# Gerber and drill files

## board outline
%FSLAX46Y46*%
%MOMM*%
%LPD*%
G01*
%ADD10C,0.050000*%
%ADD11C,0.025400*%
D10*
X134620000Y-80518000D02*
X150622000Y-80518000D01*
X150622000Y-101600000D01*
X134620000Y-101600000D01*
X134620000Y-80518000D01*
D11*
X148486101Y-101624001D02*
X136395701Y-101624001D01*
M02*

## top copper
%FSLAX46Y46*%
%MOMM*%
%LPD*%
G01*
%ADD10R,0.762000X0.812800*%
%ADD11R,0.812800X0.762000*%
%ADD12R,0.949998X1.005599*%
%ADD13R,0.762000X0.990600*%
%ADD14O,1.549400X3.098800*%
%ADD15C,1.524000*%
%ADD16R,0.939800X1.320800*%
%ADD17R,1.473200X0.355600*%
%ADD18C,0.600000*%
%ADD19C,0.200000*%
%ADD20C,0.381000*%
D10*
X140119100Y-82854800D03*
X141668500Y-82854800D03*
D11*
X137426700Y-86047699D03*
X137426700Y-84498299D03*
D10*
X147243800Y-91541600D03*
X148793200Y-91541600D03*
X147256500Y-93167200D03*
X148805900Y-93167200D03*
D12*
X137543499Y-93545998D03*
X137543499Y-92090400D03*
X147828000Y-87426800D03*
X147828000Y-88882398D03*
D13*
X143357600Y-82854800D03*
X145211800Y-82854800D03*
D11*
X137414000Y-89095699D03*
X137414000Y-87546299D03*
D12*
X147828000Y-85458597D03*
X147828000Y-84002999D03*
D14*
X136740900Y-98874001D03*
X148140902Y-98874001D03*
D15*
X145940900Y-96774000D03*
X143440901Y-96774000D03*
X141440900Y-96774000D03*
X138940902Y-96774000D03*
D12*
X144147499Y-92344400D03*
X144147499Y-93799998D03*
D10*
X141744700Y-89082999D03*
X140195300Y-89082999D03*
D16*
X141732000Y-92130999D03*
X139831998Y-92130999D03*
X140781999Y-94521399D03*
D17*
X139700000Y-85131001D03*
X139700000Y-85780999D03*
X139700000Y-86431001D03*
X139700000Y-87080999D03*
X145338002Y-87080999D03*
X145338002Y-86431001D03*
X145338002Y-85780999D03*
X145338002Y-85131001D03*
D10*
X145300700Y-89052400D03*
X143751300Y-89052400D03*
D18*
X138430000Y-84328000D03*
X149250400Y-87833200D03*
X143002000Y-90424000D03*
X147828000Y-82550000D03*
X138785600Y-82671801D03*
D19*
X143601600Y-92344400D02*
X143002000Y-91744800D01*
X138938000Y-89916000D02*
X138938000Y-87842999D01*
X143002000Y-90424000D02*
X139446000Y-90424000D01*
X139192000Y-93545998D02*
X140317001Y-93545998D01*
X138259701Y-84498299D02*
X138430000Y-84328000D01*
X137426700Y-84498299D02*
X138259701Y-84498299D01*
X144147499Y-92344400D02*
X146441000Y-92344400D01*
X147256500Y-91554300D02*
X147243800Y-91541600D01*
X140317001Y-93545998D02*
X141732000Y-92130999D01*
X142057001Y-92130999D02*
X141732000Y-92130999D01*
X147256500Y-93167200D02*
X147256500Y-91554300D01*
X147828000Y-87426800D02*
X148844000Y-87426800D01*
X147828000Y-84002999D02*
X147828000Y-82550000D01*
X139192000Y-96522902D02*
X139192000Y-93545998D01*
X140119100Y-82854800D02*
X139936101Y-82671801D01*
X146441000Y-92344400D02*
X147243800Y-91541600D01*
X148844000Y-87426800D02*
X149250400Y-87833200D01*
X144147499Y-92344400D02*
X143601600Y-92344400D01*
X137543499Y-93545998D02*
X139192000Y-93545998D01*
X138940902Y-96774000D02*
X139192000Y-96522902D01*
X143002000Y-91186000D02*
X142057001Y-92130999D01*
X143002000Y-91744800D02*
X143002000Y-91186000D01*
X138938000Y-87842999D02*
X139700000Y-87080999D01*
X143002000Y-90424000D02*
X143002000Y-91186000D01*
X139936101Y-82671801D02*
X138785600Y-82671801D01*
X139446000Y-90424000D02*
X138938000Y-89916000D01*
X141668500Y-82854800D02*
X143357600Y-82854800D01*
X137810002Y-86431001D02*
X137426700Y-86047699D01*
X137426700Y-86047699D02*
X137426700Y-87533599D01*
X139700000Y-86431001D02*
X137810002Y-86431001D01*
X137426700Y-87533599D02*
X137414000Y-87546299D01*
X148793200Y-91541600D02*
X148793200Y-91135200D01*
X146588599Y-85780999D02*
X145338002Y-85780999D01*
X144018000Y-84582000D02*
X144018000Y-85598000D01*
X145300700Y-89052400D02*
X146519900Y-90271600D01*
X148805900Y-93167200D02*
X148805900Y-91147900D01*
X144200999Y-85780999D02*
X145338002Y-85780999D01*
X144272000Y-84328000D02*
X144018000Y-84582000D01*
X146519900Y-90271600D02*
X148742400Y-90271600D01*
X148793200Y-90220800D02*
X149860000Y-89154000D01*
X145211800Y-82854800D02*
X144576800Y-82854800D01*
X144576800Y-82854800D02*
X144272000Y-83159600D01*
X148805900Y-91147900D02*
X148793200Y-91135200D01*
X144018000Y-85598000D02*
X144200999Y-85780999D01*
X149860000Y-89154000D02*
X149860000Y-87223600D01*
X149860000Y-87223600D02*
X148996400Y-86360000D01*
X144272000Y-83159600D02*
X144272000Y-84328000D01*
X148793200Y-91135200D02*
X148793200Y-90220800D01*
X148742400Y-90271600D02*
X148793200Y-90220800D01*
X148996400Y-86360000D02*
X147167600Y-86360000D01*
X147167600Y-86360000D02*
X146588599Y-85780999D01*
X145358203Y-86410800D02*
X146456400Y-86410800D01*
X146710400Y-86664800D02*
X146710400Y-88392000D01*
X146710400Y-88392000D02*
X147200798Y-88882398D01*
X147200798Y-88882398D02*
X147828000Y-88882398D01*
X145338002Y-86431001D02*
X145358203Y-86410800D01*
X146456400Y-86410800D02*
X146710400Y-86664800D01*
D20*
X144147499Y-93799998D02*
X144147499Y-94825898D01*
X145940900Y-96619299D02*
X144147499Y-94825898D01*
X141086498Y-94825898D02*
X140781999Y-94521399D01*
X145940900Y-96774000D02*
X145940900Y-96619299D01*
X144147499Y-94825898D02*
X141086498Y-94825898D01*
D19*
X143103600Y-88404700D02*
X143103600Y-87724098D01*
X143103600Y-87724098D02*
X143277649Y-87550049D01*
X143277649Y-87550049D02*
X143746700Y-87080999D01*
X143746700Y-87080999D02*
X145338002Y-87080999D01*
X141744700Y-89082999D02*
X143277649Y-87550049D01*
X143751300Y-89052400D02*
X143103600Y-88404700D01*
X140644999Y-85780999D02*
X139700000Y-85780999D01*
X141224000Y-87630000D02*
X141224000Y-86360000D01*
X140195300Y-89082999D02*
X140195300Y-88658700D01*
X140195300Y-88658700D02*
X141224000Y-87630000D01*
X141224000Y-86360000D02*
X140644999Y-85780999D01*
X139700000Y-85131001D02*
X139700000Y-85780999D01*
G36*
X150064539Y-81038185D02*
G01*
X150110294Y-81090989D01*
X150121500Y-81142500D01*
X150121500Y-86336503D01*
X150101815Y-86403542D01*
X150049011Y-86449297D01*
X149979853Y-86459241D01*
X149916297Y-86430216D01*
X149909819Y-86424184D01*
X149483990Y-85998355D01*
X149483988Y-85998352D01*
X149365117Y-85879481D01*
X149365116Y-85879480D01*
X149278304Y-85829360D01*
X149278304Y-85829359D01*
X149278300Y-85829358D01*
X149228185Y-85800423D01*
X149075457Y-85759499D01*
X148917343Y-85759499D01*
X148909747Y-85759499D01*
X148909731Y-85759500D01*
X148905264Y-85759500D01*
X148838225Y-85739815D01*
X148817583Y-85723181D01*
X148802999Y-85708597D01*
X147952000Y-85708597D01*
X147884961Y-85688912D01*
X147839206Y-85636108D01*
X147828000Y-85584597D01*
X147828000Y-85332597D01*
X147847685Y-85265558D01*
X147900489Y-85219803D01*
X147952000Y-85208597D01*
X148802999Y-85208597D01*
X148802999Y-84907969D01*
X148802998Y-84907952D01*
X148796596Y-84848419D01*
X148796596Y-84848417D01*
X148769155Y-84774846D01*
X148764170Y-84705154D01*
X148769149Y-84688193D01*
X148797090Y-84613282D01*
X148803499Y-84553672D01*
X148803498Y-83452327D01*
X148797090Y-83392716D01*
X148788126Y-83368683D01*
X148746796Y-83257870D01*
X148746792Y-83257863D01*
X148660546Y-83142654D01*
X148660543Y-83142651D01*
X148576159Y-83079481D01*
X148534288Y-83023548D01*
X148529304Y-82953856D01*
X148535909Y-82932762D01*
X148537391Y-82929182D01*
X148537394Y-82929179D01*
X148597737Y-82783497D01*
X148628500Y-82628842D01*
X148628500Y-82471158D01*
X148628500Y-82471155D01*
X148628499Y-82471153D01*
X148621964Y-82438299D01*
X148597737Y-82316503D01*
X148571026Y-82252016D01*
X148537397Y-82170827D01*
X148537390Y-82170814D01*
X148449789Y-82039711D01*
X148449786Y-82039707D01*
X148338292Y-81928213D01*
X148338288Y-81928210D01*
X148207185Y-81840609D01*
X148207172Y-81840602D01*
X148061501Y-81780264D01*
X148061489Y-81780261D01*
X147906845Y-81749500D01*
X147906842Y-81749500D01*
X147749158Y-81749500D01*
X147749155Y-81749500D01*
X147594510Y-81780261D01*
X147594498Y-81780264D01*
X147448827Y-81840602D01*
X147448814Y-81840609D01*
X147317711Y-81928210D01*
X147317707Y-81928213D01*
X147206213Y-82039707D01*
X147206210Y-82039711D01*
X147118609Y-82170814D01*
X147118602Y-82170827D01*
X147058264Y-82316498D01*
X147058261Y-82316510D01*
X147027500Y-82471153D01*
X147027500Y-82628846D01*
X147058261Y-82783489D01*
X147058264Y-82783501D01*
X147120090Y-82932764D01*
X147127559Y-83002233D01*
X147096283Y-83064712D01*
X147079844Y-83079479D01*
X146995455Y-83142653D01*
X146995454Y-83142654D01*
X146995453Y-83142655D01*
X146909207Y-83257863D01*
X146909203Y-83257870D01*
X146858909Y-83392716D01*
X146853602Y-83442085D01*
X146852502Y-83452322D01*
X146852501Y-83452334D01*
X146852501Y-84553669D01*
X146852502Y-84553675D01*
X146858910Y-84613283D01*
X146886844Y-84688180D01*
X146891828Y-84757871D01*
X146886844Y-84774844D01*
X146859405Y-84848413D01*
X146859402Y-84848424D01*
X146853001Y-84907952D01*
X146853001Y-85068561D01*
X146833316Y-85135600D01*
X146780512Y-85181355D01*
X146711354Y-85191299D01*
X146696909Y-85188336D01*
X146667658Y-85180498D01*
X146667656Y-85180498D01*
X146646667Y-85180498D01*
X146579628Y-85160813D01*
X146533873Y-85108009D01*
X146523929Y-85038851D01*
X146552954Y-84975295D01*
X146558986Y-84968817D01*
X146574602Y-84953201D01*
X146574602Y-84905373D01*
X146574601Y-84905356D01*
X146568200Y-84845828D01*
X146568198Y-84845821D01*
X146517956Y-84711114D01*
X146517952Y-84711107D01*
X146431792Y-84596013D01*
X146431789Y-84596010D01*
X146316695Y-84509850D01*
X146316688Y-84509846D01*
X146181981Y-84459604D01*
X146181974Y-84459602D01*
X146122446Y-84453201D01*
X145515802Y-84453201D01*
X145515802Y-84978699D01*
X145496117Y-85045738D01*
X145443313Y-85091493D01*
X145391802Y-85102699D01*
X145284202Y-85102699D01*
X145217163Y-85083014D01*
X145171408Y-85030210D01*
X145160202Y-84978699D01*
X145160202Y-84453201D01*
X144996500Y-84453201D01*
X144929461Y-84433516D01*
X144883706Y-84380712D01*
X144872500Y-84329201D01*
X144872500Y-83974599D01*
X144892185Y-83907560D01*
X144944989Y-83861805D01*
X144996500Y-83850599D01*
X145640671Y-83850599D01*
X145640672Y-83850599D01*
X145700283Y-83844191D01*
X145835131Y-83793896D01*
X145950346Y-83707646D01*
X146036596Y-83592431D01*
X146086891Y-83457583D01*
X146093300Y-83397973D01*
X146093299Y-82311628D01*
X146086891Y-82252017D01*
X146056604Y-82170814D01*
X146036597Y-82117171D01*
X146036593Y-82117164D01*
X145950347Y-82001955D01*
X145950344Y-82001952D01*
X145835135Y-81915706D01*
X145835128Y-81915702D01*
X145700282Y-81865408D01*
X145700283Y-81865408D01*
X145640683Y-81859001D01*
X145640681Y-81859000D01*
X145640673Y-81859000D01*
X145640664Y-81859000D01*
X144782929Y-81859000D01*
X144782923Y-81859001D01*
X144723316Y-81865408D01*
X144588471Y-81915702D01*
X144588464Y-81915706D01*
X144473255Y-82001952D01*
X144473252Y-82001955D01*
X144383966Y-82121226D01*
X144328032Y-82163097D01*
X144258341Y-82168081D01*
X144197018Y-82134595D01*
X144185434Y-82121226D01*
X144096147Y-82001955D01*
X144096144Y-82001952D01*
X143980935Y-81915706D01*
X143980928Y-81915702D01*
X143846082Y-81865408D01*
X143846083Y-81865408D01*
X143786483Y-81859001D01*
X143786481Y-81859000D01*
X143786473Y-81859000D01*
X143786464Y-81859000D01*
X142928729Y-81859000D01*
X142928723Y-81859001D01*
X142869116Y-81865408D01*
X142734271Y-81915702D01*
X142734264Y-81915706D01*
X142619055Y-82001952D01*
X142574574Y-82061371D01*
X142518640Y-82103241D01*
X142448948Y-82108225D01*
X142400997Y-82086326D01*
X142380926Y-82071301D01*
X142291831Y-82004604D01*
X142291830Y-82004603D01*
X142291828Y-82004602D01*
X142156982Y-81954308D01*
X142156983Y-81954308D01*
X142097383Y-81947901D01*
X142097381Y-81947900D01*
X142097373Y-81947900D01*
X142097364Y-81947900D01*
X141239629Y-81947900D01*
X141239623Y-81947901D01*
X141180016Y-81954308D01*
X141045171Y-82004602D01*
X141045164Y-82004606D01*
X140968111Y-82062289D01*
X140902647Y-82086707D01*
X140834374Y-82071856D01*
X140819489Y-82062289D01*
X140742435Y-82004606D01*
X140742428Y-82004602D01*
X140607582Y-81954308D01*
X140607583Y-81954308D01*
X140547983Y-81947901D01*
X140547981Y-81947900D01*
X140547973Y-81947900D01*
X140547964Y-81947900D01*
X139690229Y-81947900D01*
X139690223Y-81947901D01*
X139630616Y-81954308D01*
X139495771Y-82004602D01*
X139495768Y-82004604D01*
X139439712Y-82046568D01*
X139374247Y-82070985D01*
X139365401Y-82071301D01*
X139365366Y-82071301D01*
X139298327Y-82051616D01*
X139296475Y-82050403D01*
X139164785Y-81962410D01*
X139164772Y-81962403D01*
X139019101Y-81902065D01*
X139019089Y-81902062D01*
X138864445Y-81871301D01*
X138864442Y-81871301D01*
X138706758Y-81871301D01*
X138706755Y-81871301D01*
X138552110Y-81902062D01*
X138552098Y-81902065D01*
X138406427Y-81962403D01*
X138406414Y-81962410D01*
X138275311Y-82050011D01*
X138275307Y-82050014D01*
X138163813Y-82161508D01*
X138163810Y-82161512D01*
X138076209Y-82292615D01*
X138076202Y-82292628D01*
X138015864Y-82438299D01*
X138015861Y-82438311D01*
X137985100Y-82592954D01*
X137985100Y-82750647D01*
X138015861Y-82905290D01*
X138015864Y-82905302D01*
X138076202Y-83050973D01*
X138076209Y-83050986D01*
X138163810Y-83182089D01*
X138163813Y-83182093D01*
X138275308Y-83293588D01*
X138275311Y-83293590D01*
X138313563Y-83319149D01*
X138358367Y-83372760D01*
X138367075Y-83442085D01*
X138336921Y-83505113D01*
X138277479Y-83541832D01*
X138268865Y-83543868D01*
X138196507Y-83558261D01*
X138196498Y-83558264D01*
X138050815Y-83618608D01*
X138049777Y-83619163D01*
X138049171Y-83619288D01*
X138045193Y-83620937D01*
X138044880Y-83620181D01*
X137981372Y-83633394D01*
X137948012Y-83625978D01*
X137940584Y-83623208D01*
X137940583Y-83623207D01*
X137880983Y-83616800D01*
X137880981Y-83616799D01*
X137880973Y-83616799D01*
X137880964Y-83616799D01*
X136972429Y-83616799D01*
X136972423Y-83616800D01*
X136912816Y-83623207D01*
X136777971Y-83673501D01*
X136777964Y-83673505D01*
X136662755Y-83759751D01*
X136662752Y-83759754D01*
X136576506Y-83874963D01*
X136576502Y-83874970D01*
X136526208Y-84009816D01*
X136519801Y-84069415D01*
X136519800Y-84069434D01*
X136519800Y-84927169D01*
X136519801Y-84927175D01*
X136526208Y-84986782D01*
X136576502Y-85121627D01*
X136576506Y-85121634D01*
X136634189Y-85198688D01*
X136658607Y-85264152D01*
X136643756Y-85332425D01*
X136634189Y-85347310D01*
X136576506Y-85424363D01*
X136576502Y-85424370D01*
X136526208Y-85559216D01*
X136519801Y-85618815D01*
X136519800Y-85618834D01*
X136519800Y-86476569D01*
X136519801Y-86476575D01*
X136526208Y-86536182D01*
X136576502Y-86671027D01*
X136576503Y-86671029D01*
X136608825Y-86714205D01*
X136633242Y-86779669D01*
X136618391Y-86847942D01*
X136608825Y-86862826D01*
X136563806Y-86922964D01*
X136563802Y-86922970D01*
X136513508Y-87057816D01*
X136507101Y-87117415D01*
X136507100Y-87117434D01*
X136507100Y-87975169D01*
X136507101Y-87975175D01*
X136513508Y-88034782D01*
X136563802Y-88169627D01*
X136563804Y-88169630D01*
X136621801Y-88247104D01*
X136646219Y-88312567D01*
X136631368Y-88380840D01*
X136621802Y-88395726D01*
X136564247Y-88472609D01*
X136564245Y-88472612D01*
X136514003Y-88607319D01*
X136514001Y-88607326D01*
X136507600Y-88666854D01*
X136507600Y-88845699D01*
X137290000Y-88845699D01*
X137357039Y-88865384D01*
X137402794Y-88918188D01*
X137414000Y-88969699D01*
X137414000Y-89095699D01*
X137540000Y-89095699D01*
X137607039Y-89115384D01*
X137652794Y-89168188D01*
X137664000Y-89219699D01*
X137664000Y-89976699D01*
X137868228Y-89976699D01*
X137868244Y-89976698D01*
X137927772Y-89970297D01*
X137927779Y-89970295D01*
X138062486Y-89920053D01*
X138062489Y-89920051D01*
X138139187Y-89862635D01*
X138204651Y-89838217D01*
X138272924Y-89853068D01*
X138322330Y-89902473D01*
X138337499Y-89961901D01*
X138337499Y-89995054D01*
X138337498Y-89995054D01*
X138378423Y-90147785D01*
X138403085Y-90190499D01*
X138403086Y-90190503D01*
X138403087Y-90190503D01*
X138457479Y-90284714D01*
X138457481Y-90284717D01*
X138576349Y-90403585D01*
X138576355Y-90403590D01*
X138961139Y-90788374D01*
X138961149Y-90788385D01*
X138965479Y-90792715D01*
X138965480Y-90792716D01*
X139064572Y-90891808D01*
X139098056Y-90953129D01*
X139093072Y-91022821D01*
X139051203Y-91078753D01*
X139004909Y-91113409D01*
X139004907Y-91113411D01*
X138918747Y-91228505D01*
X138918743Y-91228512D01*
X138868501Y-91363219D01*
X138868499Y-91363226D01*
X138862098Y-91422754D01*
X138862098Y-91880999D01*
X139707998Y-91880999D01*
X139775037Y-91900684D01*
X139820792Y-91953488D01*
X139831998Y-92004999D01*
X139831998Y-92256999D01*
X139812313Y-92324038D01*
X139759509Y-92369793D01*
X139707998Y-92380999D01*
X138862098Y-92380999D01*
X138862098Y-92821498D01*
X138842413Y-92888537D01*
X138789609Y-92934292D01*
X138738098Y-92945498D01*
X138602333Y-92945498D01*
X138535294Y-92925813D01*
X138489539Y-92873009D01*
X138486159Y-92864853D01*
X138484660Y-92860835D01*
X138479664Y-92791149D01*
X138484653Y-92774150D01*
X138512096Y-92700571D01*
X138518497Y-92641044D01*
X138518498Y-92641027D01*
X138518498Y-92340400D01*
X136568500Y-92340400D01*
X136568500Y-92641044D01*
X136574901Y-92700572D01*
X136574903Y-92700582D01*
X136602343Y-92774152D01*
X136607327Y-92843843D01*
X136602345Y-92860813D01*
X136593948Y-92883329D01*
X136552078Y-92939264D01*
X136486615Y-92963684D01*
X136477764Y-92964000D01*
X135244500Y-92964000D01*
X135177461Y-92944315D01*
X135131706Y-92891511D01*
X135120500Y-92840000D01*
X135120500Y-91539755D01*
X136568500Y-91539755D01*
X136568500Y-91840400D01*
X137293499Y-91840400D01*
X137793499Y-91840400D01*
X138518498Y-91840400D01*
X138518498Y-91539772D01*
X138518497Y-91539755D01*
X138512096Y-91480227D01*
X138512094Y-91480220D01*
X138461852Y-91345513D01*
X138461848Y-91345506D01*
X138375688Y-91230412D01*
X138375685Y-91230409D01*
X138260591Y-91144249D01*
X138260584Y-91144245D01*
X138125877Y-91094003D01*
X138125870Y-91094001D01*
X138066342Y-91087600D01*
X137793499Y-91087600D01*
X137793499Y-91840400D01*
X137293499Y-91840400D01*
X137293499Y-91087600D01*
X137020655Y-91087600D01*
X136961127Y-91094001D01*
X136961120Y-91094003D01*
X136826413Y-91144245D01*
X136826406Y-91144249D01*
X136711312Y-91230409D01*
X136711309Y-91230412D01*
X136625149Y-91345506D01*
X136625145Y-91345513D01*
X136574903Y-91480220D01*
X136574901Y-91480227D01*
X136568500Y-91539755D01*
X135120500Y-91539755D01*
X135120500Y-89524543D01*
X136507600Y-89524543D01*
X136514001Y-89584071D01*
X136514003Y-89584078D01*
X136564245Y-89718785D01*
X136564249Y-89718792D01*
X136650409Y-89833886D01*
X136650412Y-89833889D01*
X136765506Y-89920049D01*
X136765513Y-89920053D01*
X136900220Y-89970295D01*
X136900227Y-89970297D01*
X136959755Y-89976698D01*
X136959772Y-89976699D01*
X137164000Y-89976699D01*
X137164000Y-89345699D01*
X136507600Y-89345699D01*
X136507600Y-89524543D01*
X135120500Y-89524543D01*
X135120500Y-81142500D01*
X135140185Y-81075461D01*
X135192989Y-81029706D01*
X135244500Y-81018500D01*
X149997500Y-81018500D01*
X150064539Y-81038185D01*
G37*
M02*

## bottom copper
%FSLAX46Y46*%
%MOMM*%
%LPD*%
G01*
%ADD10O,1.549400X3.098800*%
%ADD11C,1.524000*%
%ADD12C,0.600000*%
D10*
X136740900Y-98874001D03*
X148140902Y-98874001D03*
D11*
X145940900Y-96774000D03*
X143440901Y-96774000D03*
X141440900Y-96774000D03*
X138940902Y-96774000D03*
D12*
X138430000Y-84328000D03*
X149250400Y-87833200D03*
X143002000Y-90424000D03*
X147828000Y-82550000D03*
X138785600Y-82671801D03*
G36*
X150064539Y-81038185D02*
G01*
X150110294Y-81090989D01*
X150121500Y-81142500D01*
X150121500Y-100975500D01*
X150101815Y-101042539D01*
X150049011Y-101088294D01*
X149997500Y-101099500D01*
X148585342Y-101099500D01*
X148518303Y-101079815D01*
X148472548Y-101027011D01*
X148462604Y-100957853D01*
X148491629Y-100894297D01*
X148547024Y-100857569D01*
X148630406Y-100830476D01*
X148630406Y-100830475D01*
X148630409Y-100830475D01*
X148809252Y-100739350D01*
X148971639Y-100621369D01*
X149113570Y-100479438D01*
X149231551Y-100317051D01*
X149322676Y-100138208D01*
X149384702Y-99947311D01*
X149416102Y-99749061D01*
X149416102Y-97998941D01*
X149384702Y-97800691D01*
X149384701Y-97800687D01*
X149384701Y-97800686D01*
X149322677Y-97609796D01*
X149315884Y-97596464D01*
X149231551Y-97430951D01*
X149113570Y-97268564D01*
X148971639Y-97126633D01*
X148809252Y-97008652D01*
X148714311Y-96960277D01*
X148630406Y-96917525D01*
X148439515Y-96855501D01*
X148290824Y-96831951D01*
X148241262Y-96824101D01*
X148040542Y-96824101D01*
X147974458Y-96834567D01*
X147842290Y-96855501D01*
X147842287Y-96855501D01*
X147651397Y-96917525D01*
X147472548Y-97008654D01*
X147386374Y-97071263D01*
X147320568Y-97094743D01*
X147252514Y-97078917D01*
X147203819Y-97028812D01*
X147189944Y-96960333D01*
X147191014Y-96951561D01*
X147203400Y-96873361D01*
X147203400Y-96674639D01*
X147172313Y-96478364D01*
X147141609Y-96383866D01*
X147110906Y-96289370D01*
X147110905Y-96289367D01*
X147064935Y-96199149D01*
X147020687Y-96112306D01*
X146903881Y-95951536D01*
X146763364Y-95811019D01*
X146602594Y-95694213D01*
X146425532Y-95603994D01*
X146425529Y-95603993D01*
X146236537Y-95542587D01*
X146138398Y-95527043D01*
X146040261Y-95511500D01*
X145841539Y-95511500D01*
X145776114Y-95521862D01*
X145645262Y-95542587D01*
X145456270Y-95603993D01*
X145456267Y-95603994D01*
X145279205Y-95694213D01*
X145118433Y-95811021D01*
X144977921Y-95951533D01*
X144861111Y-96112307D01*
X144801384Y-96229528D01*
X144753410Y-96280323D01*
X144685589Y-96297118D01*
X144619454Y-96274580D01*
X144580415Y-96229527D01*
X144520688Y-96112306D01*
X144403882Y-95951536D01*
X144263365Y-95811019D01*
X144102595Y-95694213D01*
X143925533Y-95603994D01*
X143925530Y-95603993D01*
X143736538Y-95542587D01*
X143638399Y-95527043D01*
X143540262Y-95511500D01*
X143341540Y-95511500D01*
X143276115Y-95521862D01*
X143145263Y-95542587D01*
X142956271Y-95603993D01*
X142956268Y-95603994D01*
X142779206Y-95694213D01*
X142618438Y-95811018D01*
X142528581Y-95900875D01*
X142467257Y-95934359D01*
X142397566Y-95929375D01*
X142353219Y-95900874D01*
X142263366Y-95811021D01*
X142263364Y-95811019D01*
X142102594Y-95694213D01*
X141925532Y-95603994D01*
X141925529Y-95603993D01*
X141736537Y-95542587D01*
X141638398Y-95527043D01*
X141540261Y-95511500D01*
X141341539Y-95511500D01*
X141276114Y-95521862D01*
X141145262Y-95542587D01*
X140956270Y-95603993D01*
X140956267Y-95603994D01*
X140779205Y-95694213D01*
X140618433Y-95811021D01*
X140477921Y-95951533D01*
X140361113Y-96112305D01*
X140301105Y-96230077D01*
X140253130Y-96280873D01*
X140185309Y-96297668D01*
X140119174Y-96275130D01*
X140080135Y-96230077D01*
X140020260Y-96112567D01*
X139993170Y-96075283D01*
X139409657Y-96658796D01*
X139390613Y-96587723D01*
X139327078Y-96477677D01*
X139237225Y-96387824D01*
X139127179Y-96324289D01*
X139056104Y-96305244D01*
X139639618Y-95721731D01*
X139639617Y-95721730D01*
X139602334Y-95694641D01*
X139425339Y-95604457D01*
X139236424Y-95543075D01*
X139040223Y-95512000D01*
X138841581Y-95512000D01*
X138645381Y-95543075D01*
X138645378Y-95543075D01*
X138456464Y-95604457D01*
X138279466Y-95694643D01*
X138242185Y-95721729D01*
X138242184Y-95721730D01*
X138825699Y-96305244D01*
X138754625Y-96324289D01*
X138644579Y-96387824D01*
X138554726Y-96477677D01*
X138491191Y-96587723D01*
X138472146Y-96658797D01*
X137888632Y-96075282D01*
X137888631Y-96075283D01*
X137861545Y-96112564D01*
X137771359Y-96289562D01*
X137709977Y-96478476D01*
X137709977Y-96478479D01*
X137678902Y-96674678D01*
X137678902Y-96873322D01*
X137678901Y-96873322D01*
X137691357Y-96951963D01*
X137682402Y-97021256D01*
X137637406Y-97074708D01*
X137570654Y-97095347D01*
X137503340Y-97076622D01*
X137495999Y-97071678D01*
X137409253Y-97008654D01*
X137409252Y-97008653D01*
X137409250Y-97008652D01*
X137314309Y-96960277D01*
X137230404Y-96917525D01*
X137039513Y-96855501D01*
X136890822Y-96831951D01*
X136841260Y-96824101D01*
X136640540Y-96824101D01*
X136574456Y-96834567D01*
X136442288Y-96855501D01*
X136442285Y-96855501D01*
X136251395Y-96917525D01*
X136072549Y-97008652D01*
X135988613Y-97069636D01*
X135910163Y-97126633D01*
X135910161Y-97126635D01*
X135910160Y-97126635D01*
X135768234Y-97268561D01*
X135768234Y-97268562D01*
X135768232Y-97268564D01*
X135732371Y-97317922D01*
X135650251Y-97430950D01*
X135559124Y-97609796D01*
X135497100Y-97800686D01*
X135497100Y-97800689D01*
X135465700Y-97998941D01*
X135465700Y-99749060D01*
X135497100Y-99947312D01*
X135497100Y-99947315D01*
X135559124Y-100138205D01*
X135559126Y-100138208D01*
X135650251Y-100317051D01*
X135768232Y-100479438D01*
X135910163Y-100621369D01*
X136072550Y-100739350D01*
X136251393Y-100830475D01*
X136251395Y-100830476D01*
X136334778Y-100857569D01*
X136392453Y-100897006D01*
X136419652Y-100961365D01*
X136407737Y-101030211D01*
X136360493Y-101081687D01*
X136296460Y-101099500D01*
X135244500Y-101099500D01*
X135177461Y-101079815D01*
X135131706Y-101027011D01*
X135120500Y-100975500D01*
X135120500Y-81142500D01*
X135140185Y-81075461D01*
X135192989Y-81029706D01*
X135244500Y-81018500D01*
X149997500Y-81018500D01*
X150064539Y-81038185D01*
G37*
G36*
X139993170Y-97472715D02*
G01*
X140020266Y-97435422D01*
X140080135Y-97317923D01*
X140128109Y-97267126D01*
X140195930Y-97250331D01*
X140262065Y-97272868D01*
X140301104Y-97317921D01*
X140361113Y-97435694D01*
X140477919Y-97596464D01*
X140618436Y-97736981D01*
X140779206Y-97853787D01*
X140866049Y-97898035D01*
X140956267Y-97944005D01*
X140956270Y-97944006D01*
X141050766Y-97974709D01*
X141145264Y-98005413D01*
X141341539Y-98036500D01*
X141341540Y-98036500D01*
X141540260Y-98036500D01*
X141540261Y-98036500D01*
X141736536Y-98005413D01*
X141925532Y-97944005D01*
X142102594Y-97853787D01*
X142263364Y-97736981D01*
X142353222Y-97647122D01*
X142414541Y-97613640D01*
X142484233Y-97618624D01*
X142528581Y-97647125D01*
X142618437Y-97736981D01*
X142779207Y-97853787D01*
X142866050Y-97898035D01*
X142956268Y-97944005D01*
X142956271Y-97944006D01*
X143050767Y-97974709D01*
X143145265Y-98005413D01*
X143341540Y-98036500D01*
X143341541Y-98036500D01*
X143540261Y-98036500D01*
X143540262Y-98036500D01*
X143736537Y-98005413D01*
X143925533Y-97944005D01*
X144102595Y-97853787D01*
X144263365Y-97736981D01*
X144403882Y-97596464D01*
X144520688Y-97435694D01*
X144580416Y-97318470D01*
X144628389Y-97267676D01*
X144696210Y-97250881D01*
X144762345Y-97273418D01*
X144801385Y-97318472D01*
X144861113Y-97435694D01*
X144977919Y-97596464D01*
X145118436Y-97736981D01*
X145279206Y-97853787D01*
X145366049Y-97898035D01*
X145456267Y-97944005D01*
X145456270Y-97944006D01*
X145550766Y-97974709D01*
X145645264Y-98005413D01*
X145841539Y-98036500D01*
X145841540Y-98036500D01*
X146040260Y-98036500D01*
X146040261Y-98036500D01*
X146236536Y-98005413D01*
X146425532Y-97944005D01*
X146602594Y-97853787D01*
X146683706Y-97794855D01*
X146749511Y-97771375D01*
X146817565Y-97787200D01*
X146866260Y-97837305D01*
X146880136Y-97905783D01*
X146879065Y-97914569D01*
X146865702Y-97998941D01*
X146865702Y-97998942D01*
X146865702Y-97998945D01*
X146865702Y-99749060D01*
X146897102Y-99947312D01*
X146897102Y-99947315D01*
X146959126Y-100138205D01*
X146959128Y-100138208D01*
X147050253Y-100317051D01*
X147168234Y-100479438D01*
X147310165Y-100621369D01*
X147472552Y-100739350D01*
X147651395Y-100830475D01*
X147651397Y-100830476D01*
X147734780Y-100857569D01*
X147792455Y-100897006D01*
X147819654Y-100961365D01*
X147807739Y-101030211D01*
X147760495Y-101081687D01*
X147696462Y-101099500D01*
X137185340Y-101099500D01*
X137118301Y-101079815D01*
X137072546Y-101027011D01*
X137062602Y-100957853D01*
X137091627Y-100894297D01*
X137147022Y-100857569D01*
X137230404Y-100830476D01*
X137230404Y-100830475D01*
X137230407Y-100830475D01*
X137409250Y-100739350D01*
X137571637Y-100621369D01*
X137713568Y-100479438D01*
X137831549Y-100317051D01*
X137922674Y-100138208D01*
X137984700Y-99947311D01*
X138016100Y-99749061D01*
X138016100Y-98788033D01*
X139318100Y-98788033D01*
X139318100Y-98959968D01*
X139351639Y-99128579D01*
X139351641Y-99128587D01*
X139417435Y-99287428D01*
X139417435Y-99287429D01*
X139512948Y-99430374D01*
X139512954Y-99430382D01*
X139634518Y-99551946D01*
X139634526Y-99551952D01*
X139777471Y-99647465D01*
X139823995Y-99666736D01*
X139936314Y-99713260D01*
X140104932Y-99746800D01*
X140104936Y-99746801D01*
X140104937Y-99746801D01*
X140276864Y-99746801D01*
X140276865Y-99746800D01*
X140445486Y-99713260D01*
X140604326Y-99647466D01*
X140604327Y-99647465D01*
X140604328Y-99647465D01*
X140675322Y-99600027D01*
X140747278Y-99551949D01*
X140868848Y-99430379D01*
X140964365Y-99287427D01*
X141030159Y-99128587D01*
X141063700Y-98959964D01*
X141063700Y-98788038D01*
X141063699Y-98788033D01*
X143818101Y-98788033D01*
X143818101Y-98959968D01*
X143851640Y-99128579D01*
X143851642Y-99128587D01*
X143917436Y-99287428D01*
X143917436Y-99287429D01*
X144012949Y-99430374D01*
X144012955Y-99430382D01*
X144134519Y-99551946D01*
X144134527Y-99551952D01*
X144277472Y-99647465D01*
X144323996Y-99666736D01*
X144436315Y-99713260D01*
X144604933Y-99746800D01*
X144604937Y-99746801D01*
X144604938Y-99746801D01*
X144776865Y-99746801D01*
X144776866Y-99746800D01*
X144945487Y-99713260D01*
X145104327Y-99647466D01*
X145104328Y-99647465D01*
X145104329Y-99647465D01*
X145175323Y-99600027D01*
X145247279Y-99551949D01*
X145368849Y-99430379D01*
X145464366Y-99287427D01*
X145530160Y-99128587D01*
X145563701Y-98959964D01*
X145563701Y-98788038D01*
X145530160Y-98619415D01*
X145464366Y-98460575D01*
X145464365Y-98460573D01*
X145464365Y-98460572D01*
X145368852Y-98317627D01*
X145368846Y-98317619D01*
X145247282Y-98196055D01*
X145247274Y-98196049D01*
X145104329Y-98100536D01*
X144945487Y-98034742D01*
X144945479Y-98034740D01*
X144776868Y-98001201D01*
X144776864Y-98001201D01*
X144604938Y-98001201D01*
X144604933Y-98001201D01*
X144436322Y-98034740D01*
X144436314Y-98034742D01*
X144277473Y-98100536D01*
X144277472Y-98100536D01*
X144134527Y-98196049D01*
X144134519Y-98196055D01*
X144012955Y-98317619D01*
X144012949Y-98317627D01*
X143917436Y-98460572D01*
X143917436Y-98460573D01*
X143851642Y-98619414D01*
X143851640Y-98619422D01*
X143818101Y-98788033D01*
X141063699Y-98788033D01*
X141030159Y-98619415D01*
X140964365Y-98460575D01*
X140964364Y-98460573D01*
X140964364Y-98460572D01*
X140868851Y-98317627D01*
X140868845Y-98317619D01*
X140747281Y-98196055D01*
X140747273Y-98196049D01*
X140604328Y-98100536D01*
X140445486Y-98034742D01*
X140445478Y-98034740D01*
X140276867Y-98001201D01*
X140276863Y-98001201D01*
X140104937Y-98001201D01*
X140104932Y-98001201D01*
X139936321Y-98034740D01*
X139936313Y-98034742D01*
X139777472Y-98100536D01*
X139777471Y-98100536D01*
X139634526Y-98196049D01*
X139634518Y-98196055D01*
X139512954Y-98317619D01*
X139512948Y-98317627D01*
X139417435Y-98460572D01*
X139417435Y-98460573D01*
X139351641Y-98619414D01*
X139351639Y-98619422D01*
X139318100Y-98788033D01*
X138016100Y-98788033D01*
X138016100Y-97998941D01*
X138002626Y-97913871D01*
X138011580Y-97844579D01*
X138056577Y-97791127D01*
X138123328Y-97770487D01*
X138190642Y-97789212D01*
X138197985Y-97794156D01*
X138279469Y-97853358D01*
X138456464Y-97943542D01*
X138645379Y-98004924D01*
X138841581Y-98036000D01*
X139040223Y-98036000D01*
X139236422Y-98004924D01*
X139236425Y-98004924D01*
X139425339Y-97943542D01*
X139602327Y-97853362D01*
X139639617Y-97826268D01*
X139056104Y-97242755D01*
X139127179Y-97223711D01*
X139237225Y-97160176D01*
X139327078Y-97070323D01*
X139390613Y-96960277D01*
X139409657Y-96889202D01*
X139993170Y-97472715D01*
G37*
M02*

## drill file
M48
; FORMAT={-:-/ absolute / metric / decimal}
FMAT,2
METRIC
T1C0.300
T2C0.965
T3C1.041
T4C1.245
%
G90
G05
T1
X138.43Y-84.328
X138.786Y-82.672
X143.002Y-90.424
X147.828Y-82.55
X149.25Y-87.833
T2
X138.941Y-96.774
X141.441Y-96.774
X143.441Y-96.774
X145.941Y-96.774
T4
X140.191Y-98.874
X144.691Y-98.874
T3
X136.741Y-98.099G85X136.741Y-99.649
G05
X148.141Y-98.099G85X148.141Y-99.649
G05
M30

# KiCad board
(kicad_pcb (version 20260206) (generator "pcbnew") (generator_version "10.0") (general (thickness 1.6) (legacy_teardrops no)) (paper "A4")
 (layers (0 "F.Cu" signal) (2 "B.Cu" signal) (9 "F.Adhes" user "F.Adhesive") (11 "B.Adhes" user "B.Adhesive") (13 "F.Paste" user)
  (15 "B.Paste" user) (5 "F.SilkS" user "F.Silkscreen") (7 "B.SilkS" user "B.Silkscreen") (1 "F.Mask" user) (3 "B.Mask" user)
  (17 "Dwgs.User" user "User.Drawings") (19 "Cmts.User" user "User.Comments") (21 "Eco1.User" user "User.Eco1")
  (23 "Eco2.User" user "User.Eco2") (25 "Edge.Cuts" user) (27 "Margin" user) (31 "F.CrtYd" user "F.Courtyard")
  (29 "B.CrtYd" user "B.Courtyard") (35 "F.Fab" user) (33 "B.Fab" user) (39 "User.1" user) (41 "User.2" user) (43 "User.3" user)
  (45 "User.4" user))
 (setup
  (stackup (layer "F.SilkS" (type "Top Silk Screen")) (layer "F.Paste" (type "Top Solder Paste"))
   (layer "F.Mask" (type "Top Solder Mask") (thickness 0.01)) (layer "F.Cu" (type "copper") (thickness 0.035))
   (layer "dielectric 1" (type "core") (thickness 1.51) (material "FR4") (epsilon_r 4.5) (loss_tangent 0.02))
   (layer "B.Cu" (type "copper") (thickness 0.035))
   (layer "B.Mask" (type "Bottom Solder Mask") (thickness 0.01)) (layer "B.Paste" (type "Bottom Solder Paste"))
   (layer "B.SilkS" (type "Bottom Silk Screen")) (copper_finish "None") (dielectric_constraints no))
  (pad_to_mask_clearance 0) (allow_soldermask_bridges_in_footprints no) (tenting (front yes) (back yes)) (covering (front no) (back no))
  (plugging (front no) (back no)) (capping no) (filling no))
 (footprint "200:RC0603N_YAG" (layer "F.Cu") (at 140.8938 82.8548)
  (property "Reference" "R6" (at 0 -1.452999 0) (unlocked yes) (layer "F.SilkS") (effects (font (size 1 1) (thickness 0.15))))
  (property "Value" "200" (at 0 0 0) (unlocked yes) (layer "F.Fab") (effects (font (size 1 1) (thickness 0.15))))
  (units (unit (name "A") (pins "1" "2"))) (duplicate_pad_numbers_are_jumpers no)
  (pad "1" smd rect (at -0.7747 0) (size 0.762 0.8128) (layers "F.Cu" "F.Mask" "F.Paste") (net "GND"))
  (pad "2" smd rect (at 0.7747 0) (size 0.762 0.8128) (layers "F.Cu" "F.Mask" "F.Paste") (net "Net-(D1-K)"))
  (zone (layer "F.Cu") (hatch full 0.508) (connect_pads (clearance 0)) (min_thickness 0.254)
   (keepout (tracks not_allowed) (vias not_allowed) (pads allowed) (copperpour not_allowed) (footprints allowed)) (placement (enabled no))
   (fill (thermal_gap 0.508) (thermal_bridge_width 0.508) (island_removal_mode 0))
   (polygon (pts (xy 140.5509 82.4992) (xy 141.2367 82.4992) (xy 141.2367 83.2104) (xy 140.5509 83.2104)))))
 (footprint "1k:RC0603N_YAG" (layer "F.Cu") (at 137.4267 85.272999 90)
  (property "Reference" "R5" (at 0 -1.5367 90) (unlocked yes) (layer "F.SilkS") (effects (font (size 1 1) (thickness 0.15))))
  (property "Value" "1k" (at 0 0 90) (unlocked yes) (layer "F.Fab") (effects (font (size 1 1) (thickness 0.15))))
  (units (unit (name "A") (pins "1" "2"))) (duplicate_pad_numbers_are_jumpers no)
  (pad "1" smd rect (at -0.7747 0 90) (size 0.762 0.8128) (layers "F.Cu" "F.Mask" "F.Paste") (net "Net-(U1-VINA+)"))
  (pad "2" smd rect (at 0.7747 0 90) (size 0.762 0.8128) (layers "F.Cu" "F.Mask" "F.Paste") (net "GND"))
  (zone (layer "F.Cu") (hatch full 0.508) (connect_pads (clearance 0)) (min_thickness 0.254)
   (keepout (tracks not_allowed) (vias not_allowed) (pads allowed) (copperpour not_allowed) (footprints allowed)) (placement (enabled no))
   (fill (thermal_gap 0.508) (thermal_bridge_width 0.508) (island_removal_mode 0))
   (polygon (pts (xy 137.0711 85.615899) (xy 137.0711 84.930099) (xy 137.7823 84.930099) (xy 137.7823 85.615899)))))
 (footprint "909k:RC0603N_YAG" (layer "F.Cu") (at 148.0185 91.5416)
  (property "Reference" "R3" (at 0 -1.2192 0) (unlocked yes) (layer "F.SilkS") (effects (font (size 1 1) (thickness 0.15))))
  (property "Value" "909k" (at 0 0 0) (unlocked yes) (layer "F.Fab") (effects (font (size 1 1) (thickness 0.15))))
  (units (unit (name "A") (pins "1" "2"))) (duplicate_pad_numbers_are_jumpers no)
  (pad "1" smd rect (at -0.7747 0) (size 0.762 0.8128) (layers "F.Cu" "F.Mask" "F.Paste") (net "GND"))
  (pad "2" smd rect (at 0.7747 0) (size 0.762 0.8128) (layers "F.Cu" "F.Mask" "F.Paste") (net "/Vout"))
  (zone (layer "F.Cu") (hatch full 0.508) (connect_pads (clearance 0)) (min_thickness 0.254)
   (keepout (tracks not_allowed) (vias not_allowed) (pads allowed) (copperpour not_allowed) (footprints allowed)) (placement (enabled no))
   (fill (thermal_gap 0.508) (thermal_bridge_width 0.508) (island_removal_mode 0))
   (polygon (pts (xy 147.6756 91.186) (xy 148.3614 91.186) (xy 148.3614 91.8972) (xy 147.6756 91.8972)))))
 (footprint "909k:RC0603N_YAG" (layer "F.Cu") (at 148.0312 93.1672)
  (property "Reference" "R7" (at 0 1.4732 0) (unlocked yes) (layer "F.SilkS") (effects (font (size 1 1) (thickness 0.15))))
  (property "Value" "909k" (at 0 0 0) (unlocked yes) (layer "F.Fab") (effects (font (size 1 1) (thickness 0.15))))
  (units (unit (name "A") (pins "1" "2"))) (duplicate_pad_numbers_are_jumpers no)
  (pad "1" smd rect (at -0.7747 0) (size 0.762 0.8128) (layers "F.Cu" "F.Mask" "F.Paste") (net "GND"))
  (pad "2" smd rect (at 0.7747 0) (size 0.762 0.8128) (layers "F.Cu" "F.Mask" "F.Paste") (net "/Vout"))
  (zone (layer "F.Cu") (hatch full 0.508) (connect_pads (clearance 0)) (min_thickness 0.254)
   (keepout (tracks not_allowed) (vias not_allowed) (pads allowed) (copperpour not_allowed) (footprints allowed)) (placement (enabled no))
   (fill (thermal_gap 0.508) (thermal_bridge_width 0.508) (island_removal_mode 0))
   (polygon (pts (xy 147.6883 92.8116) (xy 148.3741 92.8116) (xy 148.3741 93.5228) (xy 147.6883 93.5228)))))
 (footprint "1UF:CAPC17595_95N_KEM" (layer "F.Cu") (at 137.543499 92.818199 90)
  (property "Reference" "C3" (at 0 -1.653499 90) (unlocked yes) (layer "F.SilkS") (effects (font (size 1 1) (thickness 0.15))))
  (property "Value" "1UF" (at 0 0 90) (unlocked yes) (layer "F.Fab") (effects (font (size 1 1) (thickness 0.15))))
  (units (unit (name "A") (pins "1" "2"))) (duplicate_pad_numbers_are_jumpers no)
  (pad "1" smd rect (at -0.727799 0 90) (size 1.005599 0.949998) (layers "F.Cu" "F.Mask" "F.Paste") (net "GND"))
  (pad "2" smd rect (at 0.727799 0 90) (size 1.005599 0.949998) (layers "F.Cu" "F.Mask" "F.Paste") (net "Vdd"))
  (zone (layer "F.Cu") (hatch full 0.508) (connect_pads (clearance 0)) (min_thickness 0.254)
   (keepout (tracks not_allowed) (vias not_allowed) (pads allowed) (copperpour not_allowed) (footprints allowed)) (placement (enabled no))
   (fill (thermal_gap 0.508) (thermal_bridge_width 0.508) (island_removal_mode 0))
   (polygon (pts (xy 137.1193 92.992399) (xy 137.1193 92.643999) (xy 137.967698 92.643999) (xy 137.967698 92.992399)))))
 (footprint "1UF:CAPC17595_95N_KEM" (layer "F.Cu") (at 147.828 88.154599 -90)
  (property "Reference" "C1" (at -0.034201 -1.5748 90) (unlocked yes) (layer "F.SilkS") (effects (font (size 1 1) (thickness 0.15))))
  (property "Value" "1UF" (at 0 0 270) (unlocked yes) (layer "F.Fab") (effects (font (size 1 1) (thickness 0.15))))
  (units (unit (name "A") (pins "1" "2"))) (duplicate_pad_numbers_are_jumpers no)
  (pad "1" smd rect (at -0.727799 0 270) (size 1.005599 0.949998) (layers "F.Cu" "F.Mask" "F.Paste") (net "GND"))
  (pad "2" smd rect (at 0.727799 0 270) (size 1.005599 0.949998) (layers "F.Cu" "F.Mask" "F.Paste") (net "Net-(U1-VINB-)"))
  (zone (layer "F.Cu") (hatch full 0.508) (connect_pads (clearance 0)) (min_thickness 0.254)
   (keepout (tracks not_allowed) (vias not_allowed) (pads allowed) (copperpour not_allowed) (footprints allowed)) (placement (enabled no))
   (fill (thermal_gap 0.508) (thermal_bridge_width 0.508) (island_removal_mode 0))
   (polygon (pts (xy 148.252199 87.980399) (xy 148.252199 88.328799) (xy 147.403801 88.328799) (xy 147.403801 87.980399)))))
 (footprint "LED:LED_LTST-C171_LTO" (layer "F.Cu") (at 144.2847 82.8548)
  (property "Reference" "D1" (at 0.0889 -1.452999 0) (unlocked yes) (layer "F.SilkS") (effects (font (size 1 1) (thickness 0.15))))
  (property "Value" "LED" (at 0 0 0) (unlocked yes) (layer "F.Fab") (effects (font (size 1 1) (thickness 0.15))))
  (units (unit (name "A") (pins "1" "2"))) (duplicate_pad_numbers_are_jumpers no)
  (pad "1" smd rect (at -0.9271 0) (size 0.762 0.9906) (layers "F.Cu" "F.Mask" "F.Paste") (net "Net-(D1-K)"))
  (pad "2" smd rect (at 0.9271 0) (size 0.762 0.9906) (layers "F.Cu" "F.Mask" "F.Paste") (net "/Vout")))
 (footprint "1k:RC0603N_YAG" (layer "F.Cu") (at 137.414 88.320999 90)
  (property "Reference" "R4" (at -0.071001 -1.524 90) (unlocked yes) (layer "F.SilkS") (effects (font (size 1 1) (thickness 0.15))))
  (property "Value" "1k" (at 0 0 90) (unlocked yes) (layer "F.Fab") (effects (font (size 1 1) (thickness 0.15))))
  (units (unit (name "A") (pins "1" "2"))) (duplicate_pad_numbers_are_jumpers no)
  (pad "1" smd rect (at -0.7747 0 90) (size 0.762 0.8128) (layers "F.Cu" "F.Mask" "F.Paste") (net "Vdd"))
  (pad "2" smd rect (at 0.7747 0 90) (size 0.762 0.8128) (layers "F.Cu" "F.Mask" "F.Paste") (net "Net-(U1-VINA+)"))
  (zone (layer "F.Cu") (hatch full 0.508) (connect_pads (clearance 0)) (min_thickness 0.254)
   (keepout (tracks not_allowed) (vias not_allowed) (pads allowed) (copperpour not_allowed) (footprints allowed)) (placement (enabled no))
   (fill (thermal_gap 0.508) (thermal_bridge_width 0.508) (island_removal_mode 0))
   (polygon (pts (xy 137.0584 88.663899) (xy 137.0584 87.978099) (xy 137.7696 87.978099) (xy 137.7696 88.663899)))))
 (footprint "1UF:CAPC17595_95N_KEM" (layer "F.Cu") (at 147.828 84.730798 90)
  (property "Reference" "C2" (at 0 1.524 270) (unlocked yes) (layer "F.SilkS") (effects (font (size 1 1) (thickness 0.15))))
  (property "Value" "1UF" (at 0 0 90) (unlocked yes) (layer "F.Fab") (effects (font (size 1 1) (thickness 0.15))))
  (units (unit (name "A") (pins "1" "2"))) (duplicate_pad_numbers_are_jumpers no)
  (pad "1" smd rect (at -0.727799 0 90) (size 1.005599 0.949998) (layers "F.Cu" "F.Mask" "F.Paste") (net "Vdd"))
  (pad "2" smd rect (at 0.727799 0 90) (size 1.005599 0.949998) (layers "F.Cu" "F.Mask" "F.Paste") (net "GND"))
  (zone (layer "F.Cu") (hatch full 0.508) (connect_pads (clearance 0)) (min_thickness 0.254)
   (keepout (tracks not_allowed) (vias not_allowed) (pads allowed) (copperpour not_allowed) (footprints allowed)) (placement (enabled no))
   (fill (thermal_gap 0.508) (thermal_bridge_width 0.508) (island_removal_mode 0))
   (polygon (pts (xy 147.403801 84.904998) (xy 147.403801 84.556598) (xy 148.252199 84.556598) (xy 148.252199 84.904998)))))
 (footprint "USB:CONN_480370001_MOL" (layer "F.Cu") (at 145.9409 96.774)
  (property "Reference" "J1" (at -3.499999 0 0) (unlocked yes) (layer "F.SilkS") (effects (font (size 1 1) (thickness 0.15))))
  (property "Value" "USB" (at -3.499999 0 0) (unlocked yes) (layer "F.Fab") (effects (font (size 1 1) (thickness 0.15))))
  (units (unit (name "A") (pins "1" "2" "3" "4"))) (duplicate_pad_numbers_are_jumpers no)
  (fp_line (start 2.545201 4.850001) (end -9.545199 4.850001) (stroke (width 0.0254) (type solid)) (layer "Edge.Cuts"))
  (pad "" np_thru_hole oval (at -9.2 2.100001) (size 1.5494 3.0988) (drill oval 1.0414 2.5908) (layers "*.Cu" "*.Mask"))
  (pad "" np_thru_hole circle (at -5.75 2.100001) (size 1.2446 1.2446) (drill 1.2446) (layers))
  (pad "" np_thru_hole circle (at -1.249999 2.100001) (size 1.2446 1.2446) (drill 1.2446) (layers))
  (pad "" np_thru_hole oval (at 2.200002 2.100001) (size 1.5494 3.0988) (drill oval 1.0414 2.5908) (layers "*.Cu" "*.Mask"))
  (pad "1" thru_hole circle (at 0 0) (size 1.524 1.524) (drill 0.9652) (layers "*.Cu" "*.Mask") (remove_unused_layers no) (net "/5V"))
  (pad "2" thru_hole circle (at -2.499999 0) (size 1.524 1.524) (drill 0.9652) (layers "*.Cu" "*.Mask") (remove_unused_layers no)
   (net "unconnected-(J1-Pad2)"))
  (pad "3" thru_hole circle (at -4.5 0) (size 1.524 1.524) (drill 0.9652) (layers "*.Cu" "*.Mask") (remove_unused_layers no)
   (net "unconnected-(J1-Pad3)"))
  (pad "4" thru_hole circle (at -6.999998 0) (size 1.524 1.524) (drill 0.9652) (layers "*.Cu" "*.Mask") (remove_unused_layers no)
   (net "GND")))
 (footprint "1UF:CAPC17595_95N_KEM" (layer "F.Cu") (at 144.147499 93.072199 -90)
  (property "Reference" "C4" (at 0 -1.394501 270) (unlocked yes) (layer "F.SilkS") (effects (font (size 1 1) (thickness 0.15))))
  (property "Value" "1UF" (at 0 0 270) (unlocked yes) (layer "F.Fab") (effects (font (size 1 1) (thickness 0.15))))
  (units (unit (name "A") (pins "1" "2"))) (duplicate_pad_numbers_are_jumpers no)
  (pad "1" smd rect (at -0.727799 0 270) (size 1.005599 0.949998) (layers "F.Cu" "F.Mask" "F.Paste") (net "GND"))
  (pad "2" smd rect (at 0.727799 0 270) (size 1.005599 0.949998) (layers "F.Cu" "F.Mask" "F.Paste") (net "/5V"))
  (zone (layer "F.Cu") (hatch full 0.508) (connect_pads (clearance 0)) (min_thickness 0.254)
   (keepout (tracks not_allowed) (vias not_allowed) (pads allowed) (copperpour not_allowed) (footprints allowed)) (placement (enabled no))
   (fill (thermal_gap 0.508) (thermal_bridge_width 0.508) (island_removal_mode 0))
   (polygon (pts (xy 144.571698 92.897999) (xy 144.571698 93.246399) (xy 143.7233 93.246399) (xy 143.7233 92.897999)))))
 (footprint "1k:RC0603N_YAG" (layer "F.Cu") (at 140.97 89.082999 180)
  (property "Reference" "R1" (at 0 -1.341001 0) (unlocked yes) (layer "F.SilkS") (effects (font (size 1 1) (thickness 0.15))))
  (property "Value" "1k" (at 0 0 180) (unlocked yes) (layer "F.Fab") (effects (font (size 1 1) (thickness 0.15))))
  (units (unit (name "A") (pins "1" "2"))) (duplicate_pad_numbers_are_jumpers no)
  (pad "1" smd rect (at -0.7747 0 180) (size 0.762 0.8128) (layers "F.Cu" "F.Mask" "F.Paste") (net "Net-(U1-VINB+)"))
  (pad "2" smd rect (at 0.7747 0 180) (size 0.762 0.8128) (layers "F.Cu" "F.Mask" "F.Paste") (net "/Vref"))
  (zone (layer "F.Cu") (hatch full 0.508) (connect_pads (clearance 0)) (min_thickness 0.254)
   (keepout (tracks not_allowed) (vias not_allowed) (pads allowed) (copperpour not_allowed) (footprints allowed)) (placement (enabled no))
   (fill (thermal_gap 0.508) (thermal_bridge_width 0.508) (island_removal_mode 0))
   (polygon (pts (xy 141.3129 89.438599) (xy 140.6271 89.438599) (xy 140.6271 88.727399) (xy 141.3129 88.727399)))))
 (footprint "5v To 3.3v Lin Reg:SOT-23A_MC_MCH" (layer "F.Cu") (at 140.781999 93.326199 180)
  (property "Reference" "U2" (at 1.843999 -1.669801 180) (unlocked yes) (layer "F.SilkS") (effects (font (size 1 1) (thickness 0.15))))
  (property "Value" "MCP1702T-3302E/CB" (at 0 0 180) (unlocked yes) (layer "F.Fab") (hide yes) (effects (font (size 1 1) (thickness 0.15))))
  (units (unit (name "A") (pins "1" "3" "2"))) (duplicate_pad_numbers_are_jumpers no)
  (pad "1" smd rect (at -0.950001 1.1952 180) (size 0.9398 1.3208) (layers "F.Cu" "F.Mask" "F.Paste") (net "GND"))
  (pad "2" smd rect (at 0.950001 1.1952 180) (size 0.9398 1.3208) (layers "F.Cu" "F.Mask" "F.Paste") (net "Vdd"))
  (pad "3" smd rect (at 0 -1.1952 180) (size 0.9398 1.3208) (layers "F.Cu" "F.Mask" "F.Paste") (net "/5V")))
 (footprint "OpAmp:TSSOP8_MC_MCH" (layer "F.Cu") (at 142.519001 86.106)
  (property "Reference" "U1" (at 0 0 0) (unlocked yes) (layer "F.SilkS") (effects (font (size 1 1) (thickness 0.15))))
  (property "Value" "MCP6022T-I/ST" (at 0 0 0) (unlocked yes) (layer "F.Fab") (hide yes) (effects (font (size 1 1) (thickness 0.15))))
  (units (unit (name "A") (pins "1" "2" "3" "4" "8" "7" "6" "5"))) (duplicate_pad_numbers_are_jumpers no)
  (pad "1" smd rect (at -2.819001 -0.974999) (size 1.4732 0.3556) (layers "F.Cu" "F.Mask" "F.Paste") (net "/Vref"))
  (pad "2" smd rect (at -2.819001 -0.325001) (size 1.4732 0.3556) (layers "F.Cu" "F.Mask" "F.Paste") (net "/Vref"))
  (pad "3" smd rect (at -2.819001 0.325001) (size 1.4732 0.3556) (layers "F.Cu" "F.Mask" "F.Paste") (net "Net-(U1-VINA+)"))
  (pad "4" smd rect (at -2.819001 0.974999) (size 1.4732 0.3556) (layers "F.Cu" "F.Mask" "F.Paste") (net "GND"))
  (pad "5" smd rect (at 2.819001 0.974999) (size 1.4732 0.3556) (layers "F.Cu" "F.Mask" "F.Paste") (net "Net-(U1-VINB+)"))
  (pad "6" smd rect (at 2.819001 0.325001) (size 1.4732 0.3556) (layers "F.Cu" "F.Mask" "F.Paste") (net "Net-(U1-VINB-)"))
  (pad "7" smd rect (at 2.819001 -0.325001) (size 1.4732 0.3556) (layers "F.Cu" "F.Mask" "F.Paste") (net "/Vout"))
  (pad "8" smd rect (at 2.819001 -0.974999) (size 1.4732 0.3556) (layers "F.Cu" "F.Mask" "F.Paste") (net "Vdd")))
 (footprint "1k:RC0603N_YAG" (layer "F.Cu") (at 144.526 89.0524 180)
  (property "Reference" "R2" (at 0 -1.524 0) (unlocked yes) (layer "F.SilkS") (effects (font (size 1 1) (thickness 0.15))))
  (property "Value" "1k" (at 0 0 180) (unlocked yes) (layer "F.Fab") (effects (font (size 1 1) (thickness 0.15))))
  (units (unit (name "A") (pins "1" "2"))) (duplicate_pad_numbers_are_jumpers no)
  (pad "1" smd rect (at -0.7747 0 180) (size 0.762 0.8128) (layers "F.Cu" "F.Mask" "F.Paste") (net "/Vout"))
  (pad "2" smd rect (at 0.7747 0 180) (size 0.762 0.8128) (layers "F.Cu" "F.Mask" "F.Paste") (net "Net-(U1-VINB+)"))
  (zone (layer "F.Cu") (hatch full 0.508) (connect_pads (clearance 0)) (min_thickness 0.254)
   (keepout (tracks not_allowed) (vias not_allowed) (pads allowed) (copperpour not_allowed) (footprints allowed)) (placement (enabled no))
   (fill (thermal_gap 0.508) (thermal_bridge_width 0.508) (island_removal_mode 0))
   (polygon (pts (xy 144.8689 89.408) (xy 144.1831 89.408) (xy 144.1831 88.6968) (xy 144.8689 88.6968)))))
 (gr_rect (start 134.62 80.518) (end 150.622 101.6) (stroke (width 0.05) (type default)) (fill no) (layer "Edge.Cuts"))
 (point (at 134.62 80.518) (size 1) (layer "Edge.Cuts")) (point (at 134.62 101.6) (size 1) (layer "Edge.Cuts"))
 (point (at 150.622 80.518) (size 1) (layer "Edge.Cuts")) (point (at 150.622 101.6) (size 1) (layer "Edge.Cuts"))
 (segment (start 143.6016 92.3444) (end 143.002 91.7448) (width 0.2) (layer "F.Cu") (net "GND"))
 (segment (start 138.938 89.916) (end 138.938 87.842999) (width 0.2) (layer "F.Cu") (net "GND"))
 (segment (start 143.002 90.424) (end 139.446 90.424) (width 0.2) (layer "F.Cu") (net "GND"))
 (segment (start 139.192 93.545998) (end 140.317001 93.545998) (width 0.2) (layer "F.Cu") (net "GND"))
 (segment (start 138.259701 84.498299) (end 138.43 84.328) (width 0.2) (layer "F.Cu") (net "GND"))
 (segment (start 137.4267 84.498299) (end 138.259701 84.498299) (width 0.2) (layer "F.Cu") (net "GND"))
 (segment (start 144.147499 92.3444) (end 146.441 92.3444) (width 0.2) (layer "F.Cu") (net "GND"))
 (segment (start 147.2565 91.5543) (end 147.2438 91.5416) (width 0.2) (layer "F.Cu") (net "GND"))
 (segment (start 140.317001 93.545998) (end 141.732 92.130999) (width 0.2) (layer "F.Cu") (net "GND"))
 (segment (start 142.057001 92.130999) (end 141.732 92.130999) (width 0.2) (layer "F.Cu") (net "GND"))
 (segment (start 147.2565 93.1672) (end 147.2565 91.5543) (width 0.2) (layer "F.Cu") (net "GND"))
 (segment (start 147.828 87.4268) (end 148.844 87.4268) (width 0.2) (layer "F.Cu") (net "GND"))
 (segment (start 147.828 84.002999) (end 147.828 82.55) (width 0.2) (layer "F.Cu") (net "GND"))
 (segment (start 139.192 96.522902) (end 139.192 93.545998) (width 0.2) (layer "F.Cu") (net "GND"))
 (segment (start 140.1191 82.8548) (end 139.936101 82.671801) (width 0.2) (layer "F.Cu") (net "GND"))
 (segment (start 146.441 92.3444) (end 147.2438 91.5416) (width 0.2) (layer "F.Cu") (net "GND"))
 (segment (start 148.844 87.4268) (end 149.2504 87.8332) (width 0.2) (layer "F.Cu") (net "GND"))
 (segment (start 144.147499 92.3444) (end 143.6016 92.3444) (width 0.2) (layer "F.Cu") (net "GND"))
 (segment (start 137.543499 93.545998) (end 139.192 93.545998) (width 0.2) (layer "F.Cu") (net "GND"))
 (segment (start 138.940902 96.774) (end 139.192 96.522902) (width 0.2) (layer "F.Cu") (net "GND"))
 (segment (start 143.002 91.186) (end 142.057001 92.130999) (width 0.2) (layer "F.Cu") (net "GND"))
 (segment (start 143.002 91.7448) (end 143.002 91.186) (width 0.2) (layer "F.Cu") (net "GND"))
 (segment (start 138.938 87.842999) (end 139.7 87.080999) (width 0.2) (layer "F.Cu") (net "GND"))
 (segment (start 143.002 90.424) (end 143.002 91.186) (width 0.2) (layer "F.Cu") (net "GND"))
 (segment (start 139.936101 82.671801) (end 138.7856 82.671801) (width 0.2) (layer "F.Cu") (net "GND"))
 (segment (start 139.446 90.424) (end 138.938 89.916) (width 0.2) (layer "F.Cu") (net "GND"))
 (via (at 138.43 84.328) (size 0.6) (drill 0.3) (layers "F.Cu" "B.Cu") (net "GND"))
 (via (at 149.2504 87.8332) (size 0.6) (drill 0.3) (layers "F.Cu" "B.Cu") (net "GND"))
 (via (at 143.002 90.424) (size 0.6) (drill 0.3) (layers "F.Cu" "B.Cu") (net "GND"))
 (via (at 147.828 82.55) (size 0.6) (drill 0.3) (layers "F.Cu" "B.Cu") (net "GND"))
 (via (at 138.7856 82.671801) (size 0.6) (drill 0.3) (layers "F.Cu" "B.Cu") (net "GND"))
 (segment (start 141.6685 82.8548) (end 143.3576 82.8548) (width 0.2) (layer "F.Cu") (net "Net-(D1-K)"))
 (segment (start 137.810002 86.431001) (end 137.4267 86.047699) (width 0.2) (layer "F.Cu") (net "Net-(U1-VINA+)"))
 (segment (start 137.4267 86.047699) (end 137.4267 87.533599) (width 0.2) (layer "F.Cu") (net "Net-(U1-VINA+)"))
 (segment (start 139.7 86.431001) (end 137.810002 86.431001) (width 0.2) (layer "F.Cu") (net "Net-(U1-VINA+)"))
 (segment (start 137.4267 87.533599) (end 137.414 87.546299) (width 0.2) (layer "F.Cu") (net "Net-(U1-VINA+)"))
 (segment (start 148.7932 91.5416) (end 148.7932 91.1352) (width 0.2) (layer "F.Cu") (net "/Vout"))
 (segment (start 146.588599 85.780999) (end 145.338002 85.780999) (width 0.2) (layer "F.Cu") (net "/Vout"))
 (segment (start 144.018 84.582) (end 144.018 85.598) (width 0.2) (layer "F.Cu") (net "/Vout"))
 (segment (start 145.3007 89.0524) (end 146.5199 90.2716) (width 0.2) (layer "F.Cu") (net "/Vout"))
 (segment (start 148.8059 93.1672) (end 148.8059 91.1479) (width 0.2) (layer "F.Cu") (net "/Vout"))
 (segment (start 144.200999 85.780999) (end 145.338002 85.780999) (width 0.2) (layer "F.Cu") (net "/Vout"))
 (segment (start 144.272 84.328) (end 144.018 84.582) (width 0.2) (layer "F.Cu") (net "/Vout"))
 (segment (start 146.5199 90.2716) (end 148.7424 90.2716) (width 0.2) (layer "F.Cu") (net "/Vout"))
 (segment (start 148.7932 90.2208) (end 149.86 89.154) (width 0.2) (layer "F.Cu") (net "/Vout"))
 (segment (start 145.2118 82.8548) (end 144.5768 82.8548) (width 0.2) (layer "F.Cu") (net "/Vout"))
 (segment (start 144.5768 82.8548) (end 144.272 83.1596) (width 0.2) (layer "F.Cu") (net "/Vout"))
 (segment (start 148.8059 91.1479) (end 148.7932 91.1352) (width 0.2) (layer "F.Cu") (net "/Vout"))
 (segment (start 144.018 85.598) (end 144.200999 85.780999) (width 0.2) (layer "F.Cu") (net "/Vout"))
 (segment (start 149.86 89.154) (end 149.86 87.2236) (width 0.2) (layer "F.Cu") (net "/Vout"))
 (segment (start 149.86 87.2236) (end 148.9964 86.36) (width 0.2) (layer "F.Cu") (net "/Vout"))
 (segment (start 144.272 83.1596) (end 144.272 84.328) (width 0.2) (layer "F.Cu") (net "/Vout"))
 (segment (start 148.7932 91.1352) (end 148.7932 90.2208) (width 0.2) (layer "F.Cu") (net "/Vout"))
 (segment (start 148.7424 90.2716) (end 148.7932 90.2208) (width 0.2) (layer "F.Cu") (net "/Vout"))
 (segment (start 148.9964 86.36) (end 147.1676 86.36) (width 0.2) (layer "F.Cu") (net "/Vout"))
 (segment (start 147.1676 86.36) (end 146.588599 85.780999) (width 0.2) (layer "F.Cu") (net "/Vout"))
 (segment (start 145.358203 86.4108) (end 146.4564 86.4108) (width 0.2) (layer "F.Cu") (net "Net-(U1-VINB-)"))
 (segment (start 146.7104 86.6648) (end 146.7104 88.392) (width 0.2) (layer "F.Cu") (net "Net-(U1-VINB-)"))
 (segment (start 146.7104 88.392) (end 147.200798 88.882398) (width 0.2) (layer "F.Cu") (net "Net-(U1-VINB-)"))
 (segment (start 147.200798 88.882398) (end 147.828 88.882398) (width 0.2) (layer "F.Cu") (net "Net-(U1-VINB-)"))
 (segment (start 145.338002 86.431001) (end 145.358203 86.4108) (width 0.2) (layer "F.Cu") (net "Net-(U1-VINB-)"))
 (segment (start 146.4564 86.4108) (end 146.7104 86.6648) (width 0.2) (layer "F.Cu") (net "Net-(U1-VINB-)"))
 (segment (start 144.147499 93.799998) (end 144.147499 94.825898) (width 0.381) (layer "F.Cu") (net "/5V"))
 (segment (start 145.9409 96.619299) (end 144.147499 94.825898) (width 0.381) (layer "F.Cu") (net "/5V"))
 (segment (start 141.086498 94.825898) (end 140.781999 94.521399) (width 0.381) (layer "F.Cu") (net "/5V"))
 (segment (start 145.9409 96.774) (end 145.9409 96.619299) (width 0.381) (layer "F.Cu") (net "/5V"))
 (segment (start 144.147499 94.825898) (end 141.086498 94.825898) (width 0.381) (layer "F.Cu") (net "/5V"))
 (segment (start 143.1036 88.4047) (end 143.1036 87.724098) (width 0.2) (layer "F.Cu") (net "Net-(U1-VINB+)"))
 (segment (start 143.1036 87.724098) (end 143.277649 87.550049) (width 0.2) (layer "F.Cu") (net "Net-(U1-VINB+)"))
 (segment (start 143.277649 87.550049) (end 143.7467 87.080999) (width 0.2) (layer "F.Cu") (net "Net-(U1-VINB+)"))
 (segment (start 143.7467 87.080999) (end 145.338002 87.080999) (width 0.2) (layer "F.Cu") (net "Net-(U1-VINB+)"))
 (segment (start 141.7447 89.082999) (end 143.277649 87.550049) (width 0.2) (layer "F.Cu") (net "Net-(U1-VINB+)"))
 (segment (start 143.7513 89.0524) (end 143.1036 88.4047) (width 0.2) (layer "F.Cu") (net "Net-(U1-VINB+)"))
 (segment (start 140.644999 85.780999) (end 139.7 85.780999) (width 0.2) (layer "F.Cu") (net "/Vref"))
 (segment (start 141.224 87.63) (end 141.224 86.36) (width 0.2) (layer "F.Cu") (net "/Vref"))
 (segment (start 140.1953 89.082999) (end 140.1953 88.6587) (width 0.2) (layer "F.Cu") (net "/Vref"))
 (segment (start 140.1953 88.6587) (end 141.224 87.63) (width 0.2) (layer "F.Cu") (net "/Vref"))
 (segment (start 141.224 86.36) (end 140.644999 85.780999) (width 0.2) (layer "F.Cu") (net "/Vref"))
 (segment (start 139.7 85.131001) (end 139.7 85.780999) (width 0.2) (layer "F.Cu") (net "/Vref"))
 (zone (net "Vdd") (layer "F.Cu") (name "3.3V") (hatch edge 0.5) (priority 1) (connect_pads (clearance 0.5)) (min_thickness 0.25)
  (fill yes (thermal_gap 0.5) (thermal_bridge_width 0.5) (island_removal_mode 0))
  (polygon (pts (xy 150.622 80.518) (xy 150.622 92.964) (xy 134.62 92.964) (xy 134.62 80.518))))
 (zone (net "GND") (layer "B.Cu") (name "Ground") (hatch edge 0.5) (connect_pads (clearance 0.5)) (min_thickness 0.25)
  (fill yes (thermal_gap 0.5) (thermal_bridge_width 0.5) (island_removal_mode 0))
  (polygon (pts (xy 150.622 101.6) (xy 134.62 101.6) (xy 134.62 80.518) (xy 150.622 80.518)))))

